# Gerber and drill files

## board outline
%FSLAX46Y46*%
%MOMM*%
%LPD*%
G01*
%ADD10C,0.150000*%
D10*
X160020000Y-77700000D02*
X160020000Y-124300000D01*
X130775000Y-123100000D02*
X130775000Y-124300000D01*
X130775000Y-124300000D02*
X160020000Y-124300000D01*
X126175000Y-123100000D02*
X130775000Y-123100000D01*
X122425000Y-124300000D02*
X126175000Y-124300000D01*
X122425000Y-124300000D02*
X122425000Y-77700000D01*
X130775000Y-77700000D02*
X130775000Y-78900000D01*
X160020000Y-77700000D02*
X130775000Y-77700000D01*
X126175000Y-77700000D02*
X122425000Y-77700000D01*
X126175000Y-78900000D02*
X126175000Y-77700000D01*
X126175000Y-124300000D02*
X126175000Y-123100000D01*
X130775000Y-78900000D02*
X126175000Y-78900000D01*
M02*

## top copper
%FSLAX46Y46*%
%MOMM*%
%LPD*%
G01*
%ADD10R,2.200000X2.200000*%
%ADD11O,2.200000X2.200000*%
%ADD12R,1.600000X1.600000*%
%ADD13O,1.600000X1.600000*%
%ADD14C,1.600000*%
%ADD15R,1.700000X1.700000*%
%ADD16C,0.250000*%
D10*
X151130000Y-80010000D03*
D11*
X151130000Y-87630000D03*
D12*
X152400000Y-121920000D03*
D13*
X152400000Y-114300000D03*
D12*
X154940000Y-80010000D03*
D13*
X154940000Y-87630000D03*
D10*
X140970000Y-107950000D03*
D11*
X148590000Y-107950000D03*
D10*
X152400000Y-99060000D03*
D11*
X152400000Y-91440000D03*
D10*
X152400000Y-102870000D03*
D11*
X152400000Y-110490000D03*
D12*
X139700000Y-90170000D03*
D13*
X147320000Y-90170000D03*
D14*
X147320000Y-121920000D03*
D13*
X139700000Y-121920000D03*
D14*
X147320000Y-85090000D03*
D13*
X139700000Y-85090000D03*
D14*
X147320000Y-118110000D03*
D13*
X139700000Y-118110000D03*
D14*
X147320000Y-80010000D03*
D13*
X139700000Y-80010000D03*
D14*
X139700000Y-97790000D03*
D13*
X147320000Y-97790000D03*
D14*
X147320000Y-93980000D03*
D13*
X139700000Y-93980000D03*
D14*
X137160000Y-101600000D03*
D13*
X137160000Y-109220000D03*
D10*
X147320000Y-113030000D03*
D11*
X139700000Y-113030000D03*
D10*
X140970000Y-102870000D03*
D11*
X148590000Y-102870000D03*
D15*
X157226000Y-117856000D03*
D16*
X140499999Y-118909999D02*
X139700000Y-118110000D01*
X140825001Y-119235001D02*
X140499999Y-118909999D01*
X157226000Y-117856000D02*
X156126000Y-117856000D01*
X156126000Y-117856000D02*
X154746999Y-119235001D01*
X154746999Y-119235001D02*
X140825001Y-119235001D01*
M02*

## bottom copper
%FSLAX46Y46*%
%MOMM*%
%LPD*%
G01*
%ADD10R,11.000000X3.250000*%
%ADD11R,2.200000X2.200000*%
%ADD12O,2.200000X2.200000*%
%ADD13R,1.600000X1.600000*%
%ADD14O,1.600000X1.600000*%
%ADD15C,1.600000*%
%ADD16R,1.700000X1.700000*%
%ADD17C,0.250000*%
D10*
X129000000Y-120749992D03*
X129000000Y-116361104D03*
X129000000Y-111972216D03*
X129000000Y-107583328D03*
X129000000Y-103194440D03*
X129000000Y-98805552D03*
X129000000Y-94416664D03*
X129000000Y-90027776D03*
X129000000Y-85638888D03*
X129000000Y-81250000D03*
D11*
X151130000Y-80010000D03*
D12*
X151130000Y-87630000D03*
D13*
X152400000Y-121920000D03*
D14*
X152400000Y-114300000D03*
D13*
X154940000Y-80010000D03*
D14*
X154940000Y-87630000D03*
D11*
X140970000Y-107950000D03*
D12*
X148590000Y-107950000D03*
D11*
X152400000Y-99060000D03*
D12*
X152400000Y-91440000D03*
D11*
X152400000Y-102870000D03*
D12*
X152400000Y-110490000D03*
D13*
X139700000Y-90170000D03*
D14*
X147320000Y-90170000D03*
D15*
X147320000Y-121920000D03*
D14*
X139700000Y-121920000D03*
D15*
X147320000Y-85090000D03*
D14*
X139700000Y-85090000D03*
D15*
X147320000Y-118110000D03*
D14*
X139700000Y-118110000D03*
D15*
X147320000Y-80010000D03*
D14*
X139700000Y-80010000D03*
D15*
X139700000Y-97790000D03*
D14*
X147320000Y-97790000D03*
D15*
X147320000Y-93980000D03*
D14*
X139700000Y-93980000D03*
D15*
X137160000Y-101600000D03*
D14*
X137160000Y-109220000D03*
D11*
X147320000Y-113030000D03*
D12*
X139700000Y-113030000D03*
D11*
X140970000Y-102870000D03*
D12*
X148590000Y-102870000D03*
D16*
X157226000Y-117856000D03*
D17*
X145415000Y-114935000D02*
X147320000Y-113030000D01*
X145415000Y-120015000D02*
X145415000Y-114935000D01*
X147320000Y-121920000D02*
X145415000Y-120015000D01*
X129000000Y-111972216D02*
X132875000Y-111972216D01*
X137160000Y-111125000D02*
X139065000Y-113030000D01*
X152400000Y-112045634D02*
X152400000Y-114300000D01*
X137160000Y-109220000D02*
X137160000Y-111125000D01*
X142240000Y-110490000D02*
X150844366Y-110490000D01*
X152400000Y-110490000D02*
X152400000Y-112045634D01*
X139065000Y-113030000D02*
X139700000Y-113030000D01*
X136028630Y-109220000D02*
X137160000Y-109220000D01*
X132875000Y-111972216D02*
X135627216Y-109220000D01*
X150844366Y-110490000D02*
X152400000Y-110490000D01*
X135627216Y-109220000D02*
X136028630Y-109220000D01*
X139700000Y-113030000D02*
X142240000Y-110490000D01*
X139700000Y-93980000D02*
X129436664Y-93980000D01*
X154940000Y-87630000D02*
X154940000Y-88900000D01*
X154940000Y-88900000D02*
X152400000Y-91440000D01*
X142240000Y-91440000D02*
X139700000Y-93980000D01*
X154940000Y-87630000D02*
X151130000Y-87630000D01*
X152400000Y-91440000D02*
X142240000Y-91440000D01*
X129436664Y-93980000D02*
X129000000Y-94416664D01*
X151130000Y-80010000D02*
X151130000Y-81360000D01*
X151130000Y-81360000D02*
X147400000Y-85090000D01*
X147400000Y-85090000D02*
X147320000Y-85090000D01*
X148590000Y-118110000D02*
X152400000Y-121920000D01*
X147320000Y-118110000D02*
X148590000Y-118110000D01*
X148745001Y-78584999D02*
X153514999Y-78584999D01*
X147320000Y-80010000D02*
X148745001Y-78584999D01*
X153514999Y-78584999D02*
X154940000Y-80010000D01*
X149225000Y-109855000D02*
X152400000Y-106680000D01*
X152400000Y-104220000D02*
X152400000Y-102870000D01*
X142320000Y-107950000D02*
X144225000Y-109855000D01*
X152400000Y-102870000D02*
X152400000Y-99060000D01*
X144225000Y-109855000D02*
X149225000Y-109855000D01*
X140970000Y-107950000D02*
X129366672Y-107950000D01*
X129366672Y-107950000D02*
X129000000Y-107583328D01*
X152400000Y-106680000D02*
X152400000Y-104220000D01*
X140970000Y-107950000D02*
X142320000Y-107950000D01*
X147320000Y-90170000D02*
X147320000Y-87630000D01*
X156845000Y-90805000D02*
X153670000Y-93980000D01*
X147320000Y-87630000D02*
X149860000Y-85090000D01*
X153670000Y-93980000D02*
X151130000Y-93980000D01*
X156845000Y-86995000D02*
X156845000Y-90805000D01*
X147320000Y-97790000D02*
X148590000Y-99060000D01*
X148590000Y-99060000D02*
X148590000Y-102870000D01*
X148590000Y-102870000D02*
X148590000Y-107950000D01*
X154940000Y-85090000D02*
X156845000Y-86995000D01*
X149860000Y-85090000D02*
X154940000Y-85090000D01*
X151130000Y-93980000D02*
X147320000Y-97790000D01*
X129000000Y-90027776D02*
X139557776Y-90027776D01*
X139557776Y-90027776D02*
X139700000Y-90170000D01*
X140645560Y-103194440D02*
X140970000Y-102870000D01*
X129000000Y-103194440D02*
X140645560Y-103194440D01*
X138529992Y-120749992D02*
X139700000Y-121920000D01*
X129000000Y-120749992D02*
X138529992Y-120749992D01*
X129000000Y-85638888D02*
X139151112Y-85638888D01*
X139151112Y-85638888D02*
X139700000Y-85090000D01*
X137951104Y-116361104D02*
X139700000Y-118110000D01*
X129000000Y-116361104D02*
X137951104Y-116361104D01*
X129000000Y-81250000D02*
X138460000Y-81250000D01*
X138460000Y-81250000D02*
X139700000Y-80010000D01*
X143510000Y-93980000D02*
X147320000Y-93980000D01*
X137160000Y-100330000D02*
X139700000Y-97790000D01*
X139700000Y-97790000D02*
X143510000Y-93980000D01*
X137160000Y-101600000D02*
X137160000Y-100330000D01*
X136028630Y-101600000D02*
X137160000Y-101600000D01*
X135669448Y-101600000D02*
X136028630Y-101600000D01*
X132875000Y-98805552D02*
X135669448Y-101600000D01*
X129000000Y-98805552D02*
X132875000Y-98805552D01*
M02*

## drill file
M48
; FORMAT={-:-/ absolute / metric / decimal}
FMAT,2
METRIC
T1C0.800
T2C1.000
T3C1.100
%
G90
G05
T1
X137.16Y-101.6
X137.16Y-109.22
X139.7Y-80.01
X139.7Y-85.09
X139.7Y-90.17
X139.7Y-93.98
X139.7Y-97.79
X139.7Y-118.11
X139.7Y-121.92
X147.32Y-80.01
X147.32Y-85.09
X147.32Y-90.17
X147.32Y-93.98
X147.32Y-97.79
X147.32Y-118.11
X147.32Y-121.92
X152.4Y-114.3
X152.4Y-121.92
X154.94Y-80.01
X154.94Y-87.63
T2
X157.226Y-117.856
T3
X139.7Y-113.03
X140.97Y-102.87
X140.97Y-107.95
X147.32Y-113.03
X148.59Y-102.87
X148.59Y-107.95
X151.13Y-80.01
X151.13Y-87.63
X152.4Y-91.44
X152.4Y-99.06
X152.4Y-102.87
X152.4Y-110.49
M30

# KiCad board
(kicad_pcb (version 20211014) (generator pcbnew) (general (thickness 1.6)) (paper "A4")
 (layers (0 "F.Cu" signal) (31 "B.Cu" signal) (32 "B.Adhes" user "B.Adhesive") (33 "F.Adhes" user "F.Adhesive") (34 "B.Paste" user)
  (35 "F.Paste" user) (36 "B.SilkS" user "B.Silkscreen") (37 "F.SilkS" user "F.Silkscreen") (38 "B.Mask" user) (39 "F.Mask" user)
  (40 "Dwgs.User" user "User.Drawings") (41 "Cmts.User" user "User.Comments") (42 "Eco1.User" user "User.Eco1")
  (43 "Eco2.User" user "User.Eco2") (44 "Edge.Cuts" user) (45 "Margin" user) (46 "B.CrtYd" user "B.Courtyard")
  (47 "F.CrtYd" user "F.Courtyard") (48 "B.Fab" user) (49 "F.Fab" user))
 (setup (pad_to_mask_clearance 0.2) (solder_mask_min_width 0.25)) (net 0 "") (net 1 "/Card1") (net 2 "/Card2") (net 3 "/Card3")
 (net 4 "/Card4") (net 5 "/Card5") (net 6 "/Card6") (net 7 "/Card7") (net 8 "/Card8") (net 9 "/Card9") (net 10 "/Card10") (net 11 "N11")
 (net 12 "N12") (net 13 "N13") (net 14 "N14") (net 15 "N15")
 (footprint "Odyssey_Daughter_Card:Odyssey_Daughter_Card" (layer "F.Cu") (at 129 101)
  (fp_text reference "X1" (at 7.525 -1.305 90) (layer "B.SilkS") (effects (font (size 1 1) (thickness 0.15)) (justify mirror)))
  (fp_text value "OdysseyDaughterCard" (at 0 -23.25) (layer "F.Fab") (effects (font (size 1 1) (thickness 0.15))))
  (pad "1" smd rect locked (at 0 19.749992) (size 11 3.25) (layers "B.Cu" "B.Mask") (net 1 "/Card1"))
  (pad "2" smd rect locked (at 0 15.361104) (size 11 3.25) (layers "B.Cu" "B.Mask") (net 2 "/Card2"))
  (pad "3" smd rect locked (at 0 10.972216) (size 11 3.25) (layers "B.Cu" "B.Mask") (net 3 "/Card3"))
  (pad "4" smd rect locked (at 0 6.583328) (size 11 3.25) (layers "B.Cu" "B.Mask") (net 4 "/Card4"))
  (pad "5" smd rect locked (at 0 2.19444) (size 11 3.25) (layers "B.Cu" "B.Mask") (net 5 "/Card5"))
  (pad "6" smd rect locked (at 0 -2.194448) (size 11 3.25) (layers "B.Cu" "B.Mask") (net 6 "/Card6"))
  (pad "7" smd rect locked (at 0 -6.583336) (size 11 3.25) (layers "B.Cu" "B.Mask") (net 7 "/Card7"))
  (pad "8" smd rect locked (at 0 -10.972224) (size 11 3.25) (layers "B.Cu" "B.Mask") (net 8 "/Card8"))
  (pad "9" smd rect locked (at 0 -15.361112) (size 11 3.25) (layers "B.Cu" "B.Mask") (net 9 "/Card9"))
  (pad "10" smd rect locked (at 0 -19.75) (size 11 3.25) (layers "B.Cu" "B.Mask") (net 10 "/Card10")))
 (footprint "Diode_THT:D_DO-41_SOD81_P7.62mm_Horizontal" (layer "F.Cu") (at 151.13 80.01 -90)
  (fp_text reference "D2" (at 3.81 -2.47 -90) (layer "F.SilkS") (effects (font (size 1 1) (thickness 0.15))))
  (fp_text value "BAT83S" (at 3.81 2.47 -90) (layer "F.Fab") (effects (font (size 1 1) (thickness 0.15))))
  (pad "1" thru_hole rect locked (at 0 0 270) (size 2.2 2.2) (drill 1.1) (layers *.Cu *.Mask) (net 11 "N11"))
  (pad "2" thru_hole oval locked (at 7.62 0 270) (size 2.2 2.2) (drill 1.1) (layers *.Cu *.Mask) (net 7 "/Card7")))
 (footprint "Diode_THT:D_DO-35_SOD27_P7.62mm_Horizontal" (layer "F.Cu") (at 152.4 121.92 90)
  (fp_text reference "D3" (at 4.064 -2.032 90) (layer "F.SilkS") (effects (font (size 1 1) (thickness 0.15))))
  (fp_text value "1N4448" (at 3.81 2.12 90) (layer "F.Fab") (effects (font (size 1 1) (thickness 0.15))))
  (pad "1" thru_hole rect locked (at 0 0 90) (size 1.6 1.6) (drill 0.8) (layers *.Cu *.Mask) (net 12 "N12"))
  (pad "2" thru_hole oval locked (at 7.62 0 90) (size 1.6 1.6) (drill 0.8) (layers *.Cu *.Mask) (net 3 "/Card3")))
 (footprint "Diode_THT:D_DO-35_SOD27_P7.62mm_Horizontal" (layer "F.Cu") (at 154.94 80.01 -90)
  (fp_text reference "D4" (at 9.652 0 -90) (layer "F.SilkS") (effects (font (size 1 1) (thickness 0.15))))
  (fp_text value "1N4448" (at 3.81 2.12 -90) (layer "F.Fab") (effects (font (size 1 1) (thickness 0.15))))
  (pad "1" thru_hole rect locked (at 0 0 270) (size 1.6 1.6) (drill 0.8) (layers *.Cu *.Mask) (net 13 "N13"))
  (pad "2" thru_hole oval locked (at 7.62 0 270) (size 1.6 1.6) (drill 0.8) (layers *.Cu *.Mask) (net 7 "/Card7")))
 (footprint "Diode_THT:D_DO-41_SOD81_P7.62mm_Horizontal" (layer "F.Cu") (at 140.97 107.95)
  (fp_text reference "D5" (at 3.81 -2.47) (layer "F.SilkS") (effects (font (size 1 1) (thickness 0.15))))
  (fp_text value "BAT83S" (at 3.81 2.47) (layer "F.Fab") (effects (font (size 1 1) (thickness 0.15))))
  (pad "1" thru_hole rect locked (at 0 0) (size 2.2 2.2) (drill 1.1) (layers *.Cu *.Mask) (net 4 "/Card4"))
  (pad "2" thru_hole oval locked (at 7.62 0) (size 2.2 2.2) (drill 1.1) (layers *.Cu *.Mask) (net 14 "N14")))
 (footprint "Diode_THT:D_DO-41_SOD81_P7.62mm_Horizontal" (layer "F.Cu") (at 152.4 99.06 90)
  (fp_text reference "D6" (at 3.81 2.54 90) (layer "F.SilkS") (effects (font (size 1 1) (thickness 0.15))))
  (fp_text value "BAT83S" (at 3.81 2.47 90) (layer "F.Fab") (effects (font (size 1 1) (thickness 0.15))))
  (pad "1" thru_hole rect locked (at 0 0 90) (size 2.2 2.2) (drill 1.1) (layers *.Cu *.Mask) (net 4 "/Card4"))
  (pad "2" thru_hole oval locked (at 7.62 0 90) (size 2.2 2.2) (drill 1.1) (layers *.Cu *.Mask) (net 7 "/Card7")))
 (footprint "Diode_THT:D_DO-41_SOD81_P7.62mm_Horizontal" (layer "F.Cu") (at 152.4 102.87 -90)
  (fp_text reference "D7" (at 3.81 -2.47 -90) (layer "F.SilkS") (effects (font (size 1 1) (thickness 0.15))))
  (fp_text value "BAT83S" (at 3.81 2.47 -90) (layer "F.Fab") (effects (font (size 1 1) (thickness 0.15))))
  (pad "1" thru_hole rect locked (at 0 0 270) (size 2.2 2.2) (drill 1.1) (layers *.Cu *.Mask) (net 4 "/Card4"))
  (pad "2" thru_hole oval locked (at 7.62 0 270) (size 2.2 2.2) (drill 1.1) (layers *.Cu *.Mask) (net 3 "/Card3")))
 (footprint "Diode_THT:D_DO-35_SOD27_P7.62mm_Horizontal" (layer "F.Cu") (at 139.7 90.17)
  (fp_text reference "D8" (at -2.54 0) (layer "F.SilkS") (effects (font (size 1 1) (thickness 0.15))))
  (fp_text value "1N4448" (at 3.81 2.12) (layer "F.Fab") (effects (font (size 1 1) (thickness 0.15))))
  (pad "1" thru_hole rect locked (at 0 0) (size 1.6 1.6) (drill 0.8) (layers *.Cu *.Mask) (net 8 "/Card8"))
  (pad "2" thru_hole oval locked (at 7.62 0) (size 1.6 1.6) (drill 0.8) (layers *.Cu *.Mask) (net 14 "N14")))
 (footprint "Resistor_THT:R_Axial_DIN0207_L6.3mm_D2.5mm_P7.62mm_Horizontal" (layer "F.Cu") (at 147.32 121.92 180)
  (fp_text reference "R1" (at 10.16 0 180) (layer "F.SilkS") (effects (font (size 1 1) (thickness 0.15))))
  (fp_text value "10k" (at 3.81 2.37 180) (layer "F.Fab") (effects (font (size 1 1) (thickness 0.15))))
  (pad "1" thru_hole circle locked (at 0 0 180) (size 1.6 1.6) (drill 0.8) (layers *.Cu *.Mask) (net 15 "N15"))
  (pad "2" thru_hole oval locked (at 7.62 0 180) (size 1.6 1.6) (drill 0.8) (layers *.Cu *.Mask) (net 1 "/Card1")))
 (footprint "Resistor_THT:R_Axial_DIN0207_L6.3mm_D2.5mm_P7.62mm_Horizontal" (layer "F.Cu") (at 147.32 85.09 180)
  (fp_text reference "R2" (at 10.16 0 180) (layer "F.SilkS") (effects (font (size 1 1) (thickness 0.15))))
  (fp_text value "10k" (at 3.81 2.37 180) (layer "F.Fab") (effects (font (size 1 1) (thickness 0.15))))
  (pad "1" thru_hole circle locked (at 0 0 180) (size 1.6 1.6) (drill 0.8) (layers *.Cu *.Mask) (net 11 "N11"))
  (pad "2" thru_hole oval locked (at 7.62 0 180) (size 1.6 1.6) (drill 0.8) (layers *.Cu *.Mask) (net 9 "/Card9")))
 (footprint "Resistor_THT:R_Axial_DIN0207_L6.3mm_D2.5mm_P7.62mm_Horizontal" (layer "F.Cu") (at 147.32 118.11 180)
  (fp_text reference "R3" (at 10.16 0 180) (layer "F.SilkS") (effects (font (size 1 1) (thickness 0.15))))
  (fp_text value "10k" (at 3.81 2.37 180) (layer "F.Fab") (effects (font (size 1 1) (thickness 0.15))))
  (pad "1" thru_hole circle locked (at 0 0 180) (size 1.6 1.6) (drill 0.8) (layers *.Cu *.Mask) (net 12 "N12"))
  (pad "2" thru_hole oval locked (at 7.62 0 180) (size 1.6 1.6) (drill 0.8) (layers *.Cu *.Mask) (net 2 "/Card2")))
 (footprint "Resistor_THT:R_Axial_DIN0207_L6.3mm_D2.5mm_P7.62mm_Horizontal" (layer "F.Cu") (at 147.32 80.01 180)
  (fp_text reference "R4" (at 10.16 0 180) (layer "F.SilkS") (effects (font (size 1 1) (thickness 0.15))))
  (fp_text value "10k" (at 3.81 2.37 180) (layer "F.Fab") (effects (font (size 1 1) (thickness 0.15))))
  (pad "1" thru_hole circle locked (at 0 0 180) (size 1.6 1.6) (drill 0.8) (layers *.Cu *.Mask) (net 13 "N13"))
  (pad "2" thru_hole oval locked (at 7.62 0 180) (size 1.6 1.6) (drill 0.8) (layers *.Cu *.Mask) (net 10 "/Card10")))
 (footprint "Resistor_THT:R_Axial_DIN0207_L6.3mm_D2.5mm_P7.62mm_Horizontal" (layer "F.Cu") (at 139.7 97.79)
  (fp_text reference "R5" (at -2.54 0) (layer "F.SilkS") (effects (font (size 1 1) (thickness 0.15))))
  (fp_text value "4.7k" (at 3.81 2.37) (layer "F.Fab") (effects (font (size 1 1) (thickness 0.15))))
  (pad "1" thru_hole circle locked (at 0 0) (size 1.6 1.6) (drill 0.8) (layers *.Cu *.Mask) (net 6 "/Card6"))
  (pad "2" thru_hole oval locked (at 7.62 0) (size 1.6 1.6) (drill 0.8) (layers *.Cu *.Mask) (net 14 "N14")))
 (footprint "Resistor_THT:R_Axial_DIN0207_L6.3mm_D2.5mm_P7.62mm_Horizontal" (layer "F.Cu") (at 147.32 93.98 180)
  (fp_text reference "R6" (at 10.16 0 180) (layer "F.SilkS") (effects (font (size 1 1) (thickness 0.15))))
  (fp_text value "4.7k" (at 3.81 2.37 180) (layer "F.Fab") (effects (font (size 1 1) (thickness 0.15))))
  (pad "1" thru_hole circle locked (at 0 0 180) (size 1.6 1.6) (drill 0.8) (layers *.Cu *.Mask) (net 6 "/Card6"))
  (pad "2" thru_hole oval locked (at 7.62 0 180) (size 1.6 1.6) (drill 0.8) (layers *.Cu *.Mask) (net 7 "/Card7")))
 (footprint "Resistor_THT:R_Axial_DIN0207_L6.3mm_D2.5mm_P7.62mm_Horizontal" (layer "F.Cu") (at 137.16 101.6 -90)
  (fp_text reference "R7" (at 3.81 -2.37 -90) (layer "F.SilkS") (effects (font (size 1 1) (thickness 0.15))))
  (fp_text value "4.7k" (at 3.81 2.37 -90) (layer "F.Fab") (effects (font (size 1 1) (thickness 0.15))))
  (pad "1" thru_hole circle locked (at 0 0 270) (size 1.6 1.6) (drill 0.8) (layers *.Cu *.Mask) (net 6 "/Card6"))
  (pad "2" thru_hole oval locked (at 7.62 0 270) (size 1.6 1.6) (drill 0.8) (layers *.Cu *.Mask) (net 3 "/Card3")))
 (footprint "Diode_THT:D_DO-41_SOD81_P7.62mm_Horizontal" (layer "F.Cu") (at 147.32 113.03 180)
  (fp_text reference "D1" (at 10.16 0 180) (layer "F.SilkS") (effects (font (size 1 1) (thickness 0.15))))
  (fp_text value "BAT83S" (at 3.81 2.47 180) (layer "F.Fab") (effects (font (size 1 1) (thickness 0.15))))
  (pad "1" thru_hole rect locked (at 0 0 180) (size 2.2 2.2) (drill 1.1) (layers *.Cu *.Mask) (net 15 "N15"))
  (pad "2" thru_hole oval locked (at 7.62 0 180) (size 2.2 2.2) (drill 1.1) (layers *.Cu *.Mask) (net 3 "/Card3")))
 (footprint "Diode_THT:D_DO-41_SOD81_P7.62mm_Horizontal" (layer "F.Cu") (at 140.97 102.87)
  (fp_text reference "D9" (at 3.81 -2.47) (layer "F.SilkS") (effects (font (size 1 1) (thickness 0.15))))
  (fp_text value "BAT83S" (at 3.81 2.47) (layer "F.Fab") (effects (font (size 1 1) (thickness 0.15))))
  (pad "1" thru_hole rect locked (at 0 0) (size 2.2 2.2) (drill 1.1) (layers *.Cu *.Mask) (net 5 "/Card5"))
  (pad "2" thru_hole oval locked (at 7.62 0) (size 2.2 2.2) (drill 1.1) (layers *.Cu *.Mask) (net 14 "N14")))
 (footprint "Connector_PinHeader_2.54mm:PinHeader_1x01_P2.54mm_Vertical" (layer "F.Cu") (at 157.226 117.856)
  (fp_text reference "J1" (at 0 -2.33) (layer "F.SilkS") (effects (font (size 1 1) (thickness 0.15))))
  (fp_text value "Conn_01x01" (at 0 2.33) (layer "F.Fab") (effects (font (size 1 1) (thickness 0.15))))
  (pad "1" thru_hole rect locked (at 0 0) (size 1.7 1.7) (drill 1) (layers *.Cu *.Mask) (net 2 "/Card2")))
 (gr_line (start 160.02 77.7) (end 160.02 124.3) (layer "Edge.Cuts") (width 0.15))
 (gr_line (start 130.775 123.1) (end 130.775 124.3) (layer "Edge.Cuts") (width 0.15))
 (gr_line (start 130.775 124.3) (end 160.02 124.3) (layer "Edge.Cuts") (width 0.15))
 (gr_line (start 126.175 123.1) (end 130.775 123.1) (layer "Edge.Cuts") (width 0.15))
 (gr_line (start 122.425 124.3) (end 126.175 124.3) (layer "Edge.Cuts") (width 0.15))
 (gr_line (start 122.425 124.3) (end 122.425 77.7) (layer "Edge.Cuts") (width 0.15))
 (gr_line (start 130.775 77.7) (end 130.775 78.9) (layer "Edge.Cuts") (width 0.15))
 (gr_line (start 160.02 77.7) (end 130.775 77.7) (layer "Edge.Cuts") (width 0.15))
 (gr_line (start 126.175 77.7) (end 122.425 77.7) (layer "Edge.Cuts") (width 0.15))
 (gr_line (start 126.175 78.9) (end 126.175 77.7) (layer "Edge.Cuts") (width 0.15))
 (gr_line (start 126.175 124.3) (end 126.175 123.1) (layer "Edge.Cuts") (width 0.15))
 (gr_line (start 130.775 78.9) (end 126.175 78.9) (layer "Edge.Cuts") (width 0.15))
 (segment (start 145.415 114.935) (end 147.32 113.03) (width 0.25) (layer "B.Cu") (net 15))
 (segment (start 145.415 120.015) (end 145.415 114.935) (width 0.25) (layer "B.Cu") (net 15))
 (segment (start 147.32 121.92) (end 145.415 120.015) (width 0.25) (layer "B.Cu") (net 15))
 (segment (start 129 111.972216) (end 132.875 111.972216) (width 0.25) (layer "B.Cu") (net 3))
 (segment (start 137.16 111.125) (end 139.065 113.03) (width 0.25) (layer "B.Cu") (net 3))
 (segment (start 152.4 112.045634) (end 152.4 114.3) (width 0.25) (layer "B.Cu") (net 3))
 (segment (start 137.16 109.22) (end 137.16 111.125) (width 0.25) (layer "B.Cu") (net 3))
 (segment (start 142.24 110.49) (end 150.844366 110.49) (width 0.25) (layer "B.Cu") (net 3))
 (segment (start 152.4 110.49) (end 152.4 112.045634) (width 0.25) (layer "B.Cu") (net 3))
 (segment (start 139.065 113.03) (end 139.7 113.03) (width 0.25) (layer "B.Cu") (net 3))
 (segment (start 136.02863 109.22) (end 137.16 109.22) (width 0.25) (layer "B.Cu") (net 3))
 (segment (start 132.875 111.972216) (end 135.627216 109.22) (width 0.25) (layer "B.Cu") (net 3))
 (segment (start 150.844366 110.49) (end 152.4 110.49) (width 0.25) (layer "B.Cu") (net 3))
 (segment (start 135.627216 109.22) (end 136.02863 109.22) (width 0.25) (layer "B.Cu") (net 3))
 (segment (start 139.7 113.03) (end 142.24 110.49) (width 0.25) (layer "B.Cu") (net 3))
 (segment (start 139.7 93.98) (end 129.436664 93.98) (width 0.25) (layer "B.Cu") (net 7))
 (segment (start 154.94 87.63) (end 154.94 88.9) (width 0.25) (layer "B.Cu") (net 7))
 (segment (start 154.94 88.9) (end 152.4 91.44) (width 0.25) (layer "B.Cu") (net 7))
 (segment (start 142.24 91.44) (end 139.7 93.98) (width 0.25) (layer "B.Cu") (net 7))
 (segment (start 154.94 87.63) (end 151.13 87.63) (width 0.25) (layer "B.Cu") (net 7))
 (segment (start 152.4 91.44) (end 142.24 91.44) (width 0.25) (layer "B.Cu") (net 7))
 (segment (start 129.436664 93.98) (end 129 94.416664) (width 0.25) (layer "B.Cu") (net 7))
 (segment (start 151.13 80.01) (end 151.13 81.36) (width 0.25) (layer "B.Cu") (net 11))
 (segment (start 151.13 81.36) (end 147.4 85.09) (width 0.25) (layer "B.Cu") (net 11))
 (segment (start 147.4 85.09) (end 147.32 85.09) (width 0.25) (layer "B.Cu") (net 11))
 (segment (start 148.59 118.11) (end 152.4 121.92) (width 0.25) (layer "B.Cu") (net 12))
 (segment (start 147.32 118.11) (end 148.59 118.11) (width 0.25) (layer "B.Cu") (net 12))
 (segment (start 148.745001 78.584999) (end 153.514999 78.584999) (width 0.25) (layer "B.Cu") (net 13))
 (segment (start 147.32 80.01) (end 148.745001 78.584999) (width 0.25) (layer "B.Cu") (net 13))
 (segment (start 153.514999 78.584999) (end 154.94 80.01) (width 0.25) (layer "B.Cu") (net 13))
 (segment (start 149.225 109.855) (end 152.4 106.68) (width 0.25) (layer "B.Cu") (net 4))
 (segment (start 152.4 104.22) (end 152.4 102.87) (width 0.25) (layer "B.Cu") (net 4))
 (segment (start 142.32 107.95) (end 144.225 109.855) (width 0.25) (layer "B.Cu") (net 4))
 (segment (start 152.4 102.87) (end 152.4 99.06) (width 0.25) (layer "B.Cu") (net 4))
 (segment (start 144.225 109.855) (end 149.225 109.855) (width 0.25) (layer "B.Cu") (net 4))
 (segment (start 140.97 107.95) (end 129.366672 107.95) (width 0.25) (layer "B.Cu") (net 4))
 (segment (start 129.366672 107.95) (end 129 107.583328) (width 0.25) (layer "B.Cu") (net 4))
 (segment (start 152.4 106.68) (end 152.4 104.22) (width 0.25) (layer "B.Cu") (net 4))
 (segment (start 140.97 107.95) (end 142.32 107.95) (width 0.25) (layer "B.Cu") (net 4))
 (segment (start 147.32 90.17) (end 147.32 87.63) (width 0.25) (layer "B.Cu") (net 14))
 (segment (start 156.845 90.805) (end 153.67 93.98) (width 0.25) (layer "B.Cu") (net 14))
 (segment (start 147.32 87.63) (end 149.86 85.09) (width 0.25) (layer "B.Cu") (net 14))
 (segment (start 153.67 93.98) (end 151.13 93.98) (width 0.25) (layer "B.Cu") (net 14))
 (segment (start 156.845 86.995) (end 156.845 90.805) (width 0.25) (layer "B.Cu") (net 14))
 (segment (start 147.32 97.79) (end 148.59 99.06) (width 0.25) (layer "B.Cu") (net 14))
 (segment (start 148.59 99.06) (end 148.59 102.87) (width 0.25) (layer "B.Cu") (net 14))
 (segment (start 148.59 102.87) (end 148.59 107.95) (width 0.25) (layer "B.Cu") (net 14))
 (segment (start 154.94 85.09) (end 156.845 86.995) (width 0.25) (layer "B.Cu") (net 14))
 (segment (start 149.86 85.09) (end 154.94 85.09) (width 0.25) (layer "B.Cu") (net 14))
 (segment (start 151.13 93.98) (end 147.32 97.79) (width 0.25) (layer "B.Cu") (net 14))
 (segment (start 129 90.027776) (end 139.557776 90.027776) (width 0.25) (layer "B.Cu") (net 8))
 (segment (start 139.557776 90.027776) (end 139.7 90.17) (width 0.25) (layer "B.Cu") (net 8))
 (segment (start 140.64556 103.19444) (end 140.97 102.87) (width 0.25) (layer "B.Cu") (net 5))
 (segment (start 129 103.19444) (end 140.64556 103.19444) (width 0.25) (layer "B.Cu") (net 5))
 (segment (start 138.529992 120.749992) (end 139.7 121.92) (width 0.25) (layer "B.Cu") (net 1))
 (segment (start 129 120.749992) (end 138.529992 120.749992) (width 0.25) (layer "B.Cu") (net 1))
 (segment (start 129 85.638888) (end 139.151112 85.638888) (width 0.25) (layer "B.Cu") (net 9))
 (segment (start 139.151112 85.638888) (end 139.7 85.09) (width 0.25) (layer "B.Cu") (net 9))
 (segment (start 140.499999 118.909999) (end 139.7 118.11) (width 0.25) (layer "F.Cu") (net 2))
 (segment (start 140.825001 119.235001) (end 140.499999 118.909999) (width 0.25) (layer "F.Cu") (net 2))
 (segment (start 157.226 117.856) (end 156.126 117.856) (width 0.25) (layer "F.Cu") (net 2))
 (segment (start 156.126 117.856) (end 154.746999 119.235001) (width 0.25) (layer "F.Cu") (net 2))
 (segment (start 154.746999 119.235001) (end 140.825001 119.235001) (width 0.25) (layer "F.Cu") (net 2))
 (segment (start 137.951104 116.361104) (end 139.7 118.11) (width 0.25) (layer "B.Cu") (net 2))
 (segment (start 129 116.361104) (end 137.951104 116.361104) (width 0.25) (layer "B.Cu") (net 2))
 (segment (start 129 81.25) (end 138.46 81.25) (width 0.25) (layer "B.Cu") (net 10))
 (segment (start 138.46 81.25) (end 139.7 80.01) (width 0.25) (layer "B.Cu") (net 10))
 (segment (start 143.51 93.98) (end 147.32 93.98) (width 0.25) (layer "B.Cu") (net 6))
 (segment (start 137.16 100.33) (end 139.7 97.79) (width 0.25) (layer "B.Cu") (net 6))
 (segment (start 139.7 97.79) (end 143.51 93.98) (width 0.25) (layer "B.Cu") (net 6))
 (segment (start 137.16 101.6) (end 137.16 100.33) (width 0.25) (layer "B.Cu") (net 6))
 (segment (start 136.02863 101.6) (end 137.16 101.6) (width 0.25) (layer "B.Cu") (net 6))
 (segment (start 135.669448 101.6) (end 136.02863 101.6) (width 0.25) (layer "B.Cu") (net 6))
 (segment (start 132.875 98.805552) (end 135.669448 101.6) (width 0.25) (layer "B.Cu") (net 6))
 (segment (start 129 98.805552) (end 132.875 98.805552) (width 0.25) (layer "B.Cu") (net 6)))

